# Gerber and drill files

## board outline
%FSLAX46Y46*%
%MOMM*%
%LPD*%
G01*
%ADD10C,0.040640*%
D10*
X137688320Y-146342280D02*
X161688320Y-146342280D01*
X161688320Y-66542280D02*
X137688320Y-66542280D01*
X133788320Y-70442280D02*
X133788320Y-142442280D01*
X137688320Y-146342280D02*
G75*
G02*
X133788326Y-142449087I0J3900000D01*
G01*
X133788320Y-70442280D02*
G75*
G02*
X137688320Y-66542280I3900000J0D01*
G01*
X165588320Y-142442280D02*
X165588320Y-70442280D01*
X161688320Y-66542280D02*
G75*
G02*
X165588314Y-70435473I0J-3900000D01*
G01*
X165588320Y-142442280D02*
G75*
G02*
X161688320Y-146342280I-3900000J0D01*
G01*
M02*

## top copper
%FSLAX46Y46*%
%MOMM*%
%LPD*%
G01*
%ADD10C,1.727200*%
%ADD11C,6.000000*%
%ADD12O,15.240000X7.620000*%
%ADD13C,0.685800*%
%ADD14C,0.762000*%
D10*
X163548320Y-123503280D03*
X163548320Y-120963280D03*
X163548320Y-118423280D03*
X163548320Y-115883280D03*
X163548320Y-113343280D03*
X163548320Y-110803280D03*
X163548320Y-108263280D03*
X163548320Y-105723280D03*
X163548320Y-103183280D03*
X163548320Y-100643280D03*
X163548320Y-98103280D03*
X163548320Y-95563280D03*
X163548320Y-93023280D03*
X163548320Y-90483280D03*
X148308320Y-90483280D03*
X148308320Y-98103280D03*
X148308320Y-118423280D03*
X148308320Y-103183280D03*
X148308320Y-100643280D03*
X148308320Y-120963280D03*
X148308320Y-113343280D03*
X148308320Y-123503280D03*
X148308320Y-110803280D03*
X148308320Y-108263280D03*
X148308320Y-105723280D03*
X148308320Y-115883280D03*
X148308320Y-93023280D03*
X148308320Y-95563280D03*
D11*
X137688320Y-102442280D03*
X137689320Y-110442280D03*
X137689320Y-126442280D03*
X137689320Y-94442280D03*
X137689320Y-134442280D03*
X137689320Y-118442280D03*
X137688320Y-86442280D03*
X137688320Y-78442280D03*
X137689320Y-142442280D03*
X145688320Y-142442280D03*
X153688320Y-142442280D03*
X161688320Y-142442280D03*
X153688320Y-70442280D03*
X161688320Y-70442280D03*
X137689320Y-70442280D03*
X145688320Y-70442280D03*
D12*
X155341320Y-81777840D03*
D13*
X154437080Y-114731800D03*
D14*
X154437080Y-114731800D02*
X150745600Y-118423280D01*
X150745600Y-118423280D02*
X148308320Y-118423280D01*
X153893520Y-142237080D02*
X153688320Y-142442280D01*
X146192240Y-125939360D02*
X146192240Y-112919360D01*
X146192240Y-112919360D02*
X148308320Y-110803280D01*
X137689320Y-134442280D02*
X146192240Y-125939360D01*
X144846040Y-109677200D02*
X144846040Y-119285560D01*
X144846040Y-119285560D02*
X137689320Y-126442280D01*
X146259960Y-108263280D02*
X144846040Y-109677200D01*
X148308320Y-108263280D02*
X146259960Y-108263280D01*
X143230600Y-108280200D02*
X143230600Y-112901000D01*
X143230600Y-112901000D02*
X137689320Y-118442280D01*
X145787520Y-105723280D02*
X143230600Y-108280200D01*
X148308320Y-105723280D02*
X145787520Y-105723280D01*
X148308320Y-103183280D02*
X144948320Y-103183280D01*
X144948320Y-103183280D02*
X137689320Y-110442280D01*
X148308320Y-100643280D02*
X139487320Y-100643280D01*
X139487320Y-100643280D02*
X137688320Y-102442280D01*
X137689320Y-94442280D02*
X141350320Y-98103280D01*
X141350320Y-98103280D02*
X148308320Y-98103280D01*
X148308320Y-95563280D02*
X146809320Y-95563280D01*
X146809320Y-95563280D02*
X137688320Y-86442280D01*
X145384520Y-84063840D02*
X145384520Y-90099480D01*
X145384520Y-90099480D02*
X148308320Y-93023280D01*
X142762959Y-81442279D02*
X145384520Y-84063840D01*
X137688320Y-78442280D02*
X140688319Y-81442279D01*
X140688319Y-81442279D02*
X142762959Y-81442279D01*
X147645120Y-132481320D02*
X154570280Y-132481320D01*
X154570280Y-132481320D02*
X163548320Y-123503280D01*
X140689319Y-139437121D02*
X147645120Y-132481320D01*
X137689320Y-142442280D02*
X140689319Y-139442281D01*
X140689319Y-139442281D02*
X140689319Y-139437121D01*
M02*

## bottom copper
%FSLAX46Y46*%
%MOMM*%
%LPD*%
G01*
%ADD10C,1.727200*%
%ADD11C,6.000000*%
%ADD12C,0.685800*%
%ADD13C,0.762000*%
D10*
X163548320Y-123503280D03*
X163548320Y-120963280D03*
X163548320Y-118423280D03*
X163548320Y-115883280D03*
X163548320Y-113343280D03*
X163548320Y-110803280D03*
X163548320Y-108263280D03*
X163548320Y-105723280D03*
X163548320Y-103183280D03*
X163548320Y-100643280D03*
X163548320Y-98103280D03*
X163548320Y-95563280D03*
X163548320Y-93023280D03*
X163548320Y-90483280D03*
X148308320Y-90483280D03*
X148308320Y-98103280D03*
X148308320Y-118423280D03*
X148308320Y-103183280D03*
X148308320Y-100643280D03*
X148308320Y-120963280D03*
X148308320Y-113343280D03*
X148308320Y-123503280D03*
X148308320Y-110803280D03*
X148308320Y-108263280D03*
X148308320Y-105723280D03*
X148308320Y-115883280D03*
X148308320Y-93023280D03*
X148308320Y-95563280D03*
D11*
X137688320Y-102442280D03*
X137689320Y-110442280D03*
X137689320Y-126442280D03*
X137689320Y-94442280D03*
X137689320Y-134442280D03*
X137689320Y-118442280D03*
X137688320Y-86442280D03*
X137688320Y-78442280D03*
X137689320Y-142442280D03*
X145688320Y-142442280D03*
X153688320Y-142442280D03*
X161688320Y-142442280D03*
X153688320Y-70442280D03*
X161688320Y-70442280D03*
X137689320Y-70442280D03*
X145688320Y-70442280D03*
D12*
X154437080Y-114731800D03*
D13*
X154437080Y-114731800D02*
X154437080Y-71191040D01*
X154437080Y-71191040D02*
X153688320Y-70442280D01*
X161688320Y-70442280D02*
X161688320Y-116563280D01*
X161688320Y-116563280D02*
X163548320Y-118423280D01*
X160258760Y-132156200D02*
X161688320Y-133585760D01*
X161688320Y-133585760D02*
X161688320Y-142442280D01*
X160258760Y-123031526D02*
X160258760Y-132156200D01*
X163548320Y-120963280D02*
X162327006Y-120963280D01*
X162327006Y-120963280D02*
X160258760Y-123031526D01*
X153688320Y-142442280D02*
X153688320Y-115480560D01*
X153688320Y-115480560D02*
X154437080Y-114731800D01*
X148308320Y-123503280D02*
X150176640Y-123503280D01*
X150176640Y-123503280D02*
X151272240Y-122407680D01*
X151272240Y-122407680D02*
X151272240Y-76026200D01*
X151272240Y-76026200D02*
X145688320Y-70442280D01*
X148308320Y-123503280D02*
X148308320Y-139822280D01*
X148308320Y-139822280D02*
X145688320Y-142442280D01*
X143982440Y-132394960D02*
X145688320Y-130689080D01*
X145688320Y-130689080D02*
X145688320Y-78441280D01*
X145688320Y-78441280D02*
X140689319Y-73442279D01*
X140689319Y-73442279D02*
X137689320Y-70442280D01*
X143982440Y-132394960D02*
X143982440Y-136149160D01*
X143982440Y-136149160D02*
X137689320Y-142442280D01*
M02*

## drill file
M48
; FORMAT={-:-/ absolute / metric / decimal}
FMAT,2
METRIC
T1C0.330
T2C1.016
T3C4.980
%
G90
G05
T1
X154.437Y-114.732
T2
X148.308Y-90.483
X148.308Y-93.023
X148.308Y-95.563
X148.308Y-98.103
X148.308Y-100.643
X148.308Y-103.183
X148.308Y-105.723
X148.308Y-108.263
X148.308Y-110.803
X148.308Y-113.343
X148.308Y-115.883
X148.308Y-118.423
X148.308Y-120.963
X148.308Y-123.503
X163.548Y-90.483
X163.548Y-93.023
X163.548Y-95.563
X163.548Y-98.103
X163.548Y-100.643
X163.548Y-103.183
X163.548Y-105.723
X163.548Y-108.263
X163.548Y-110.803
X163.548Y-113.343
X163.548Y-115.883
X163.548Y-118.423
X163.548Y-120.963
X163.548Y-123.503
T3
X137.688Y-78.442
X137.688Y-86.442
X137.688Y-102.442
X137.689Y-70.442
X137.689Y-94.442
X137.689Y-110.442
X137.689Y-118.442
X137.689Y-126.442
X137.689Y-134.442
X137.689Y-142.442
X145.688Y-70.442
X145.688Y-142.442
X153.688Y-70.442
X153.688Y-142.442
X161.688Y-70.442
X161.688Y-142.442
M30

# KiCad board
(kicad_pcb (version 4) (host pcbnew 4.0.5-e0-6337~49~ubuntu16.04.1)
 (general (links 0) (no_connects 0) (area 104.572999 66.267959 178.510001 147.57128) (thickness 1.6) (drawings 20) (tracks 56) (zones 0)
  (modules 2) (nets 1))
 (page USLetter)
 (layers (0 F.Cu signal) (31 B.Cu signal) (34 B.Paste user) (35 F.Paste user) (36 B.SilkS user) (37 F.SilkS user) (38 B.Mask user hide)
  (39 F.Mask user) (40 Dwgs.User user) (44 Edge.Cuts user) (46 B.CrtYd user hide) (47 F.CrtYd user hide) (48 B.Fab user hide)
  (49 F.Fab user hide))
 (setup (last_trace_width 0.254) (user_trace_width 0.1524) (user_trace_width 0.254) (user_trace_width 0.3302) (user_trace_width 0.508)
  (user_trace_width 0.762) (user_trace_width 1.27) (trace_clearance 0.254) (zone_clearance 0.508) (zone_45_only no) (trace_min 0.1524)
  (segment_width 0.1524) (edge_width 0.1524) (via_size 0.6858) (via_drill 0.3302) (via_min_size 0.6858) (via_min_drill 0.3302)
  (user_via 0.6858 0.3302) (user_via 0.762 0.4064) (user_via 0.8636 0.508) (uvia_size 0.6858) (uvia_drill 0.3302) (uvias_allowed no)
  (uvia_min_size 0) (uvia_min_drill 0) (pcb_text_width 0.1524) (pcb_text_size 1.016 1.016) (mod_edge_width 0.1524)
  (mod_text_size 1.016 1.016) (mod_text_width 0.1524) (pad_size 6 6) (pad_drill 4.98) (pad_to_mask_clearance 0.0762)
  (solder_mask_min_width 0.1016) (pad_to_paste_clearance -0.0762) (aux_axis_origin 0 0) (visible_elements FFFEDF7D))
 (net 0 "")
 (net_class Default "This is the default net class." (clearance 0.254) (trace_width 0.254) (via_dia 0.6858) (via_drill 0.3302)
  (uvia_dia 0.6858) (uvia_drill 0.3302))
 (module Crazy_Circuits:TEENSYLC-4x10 (layer F.Cu) (at 137.68832 94.44228)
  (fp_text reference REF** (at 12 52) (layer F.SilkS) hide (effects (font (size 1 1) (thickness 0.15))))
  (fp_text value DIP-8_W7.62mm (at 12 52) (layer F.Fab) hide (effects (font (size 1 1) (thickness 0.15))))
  (fp_line (start 0 51.9) (end 24 51.9) (layer Edge.Cuts) (width 0.04064))
  (fp_line (start 24 -27.9) (end 0 -27.9) (layer Edge.Cuts) (width 0.04064))
  (fp_line (start -3.9 -24) (end -3.9 48) (layer Edge.Cuts) (width 0.04064))
  (fp_arc (start 0 48) (end 0 51.9) (angle 89.9) (layer Edge.Cuts) (width 0.04064))
  (fp_arc (start 0 -24) (end -3.9 -24) (angle 90) (layer Edge.Cuts) (width 0.04064))
  (fp_line (start 27.9 48) (end 27.9 -24) (layer Edge.Cuts) (width 0.04064))
  (fp_arc (start 24 -24) (end 24 -27.9) (angle 89.9) (layer Edge.Cuts) (width 0.04064))
  (fp_arc (start 24 48) (end 27.9 48) (angle 90) (layer Edge.Cuts) (width 0.04064))
  (pad GND thru_hole circle (at 25.86 29.061 180) (size 1.7272 1.7272) (drill 1.016) (layers *.Cu *.Mask F.SilkS))
  (pad 0 thru_hole circle (at 25.86 26.521 180) (size 1.7272 1.7272) (drill 1.016) (layers *.Cu *.Mask F.SilkS))
  (pad 1 thru_hole circle (at 25.86 23.981 180) (size 1.7272 1.7272) (drill 1.016) (layers *.Cu *.Mask F.SilkS))
  (pad 2 thru_hole circle (at 25.86 21.441 180) (size 1.7272 1.7272) (drill 1.016) (layers *.Cu *.Mask F.SilkS))
  (pad 3 thru_hole circle (at 25.86 18.901 180) (size 1.7272 1.7272) (drill 1.016) (layers *.Cu *.Mask F.SilkS))
  (pad 4 thru_hole circle (at 25.86 16.361 180) (size 1.7272 1.7272) (drill 1.016) (layers *.Cu *.Mask F.SilkS))
  (pad 5 thru_hole circle (at 25.86 13.821 180) (size 1.7272 1.7272) (drill 1.016) (layers *.Cu *.Mask F.SilkS))
  (pad 6 thru_hole circle (at 25.86 11.281 180) (size 1.7272 1.7272) (drill 1.016) (layers *.Cu *.Mask F.SilkS))
  (pad 7 thru_hole circle (at 25.86 8.741 180) (size 1.7272 1.7272) (drill 1.016) (layers *.Cu *.Mask F.SilkS))
  (pad 8 thru_hole circle (at 25.86 6.201 180) (size 1.7272 1.7272) (drill 1.016) (layers *.Cu *.Mask F.SilkS))
  (pad 9 thru_hole circle (at 25.86 3.661 180) (size 1.7272 1.7272) (drill 1.016) (layers *.Cu *.Mask F.SilkS))
  (pad 10 thru_hole circle (at 25.86 1.121 180) (size 1.7272 1.7272) (drill 1.016) (layers *.Cu *.Mask F.SilkS))
  (pad 11 thru_hole circle (at 25.86 -1.419 180) (size 1.7272 1.7272) (drill 1.016) (layers *.Cu *.Mask F.SilkS))
  (pad 12 thru_hole circle (at 25.86 -3.959 180) (size 1.7272 1.7272) (drill 1.016) (layers *.Cu *.Mask F.SilkS))
  (pad 13 thru_hole circle (at 10.62 -3.959 180) (size 1.7272 1.7272) (drill 1.016) (layers *.Cu *.Mask F.SilkS))
  (pad 16 thru_hole circle (at 10.62 3.661 180) (size 1.7272 1.7272) (drill 1.016) (layers *.Cu *.Mask F.SilkS))
  (pad 3.3V thru_hole circle (at 10.62 23.981 180) (size 1.7272 1.7272) (drill 1.016) (layers *.Cu *.Mask F.SilkS))
  (pad 18 thru_hole circle (at 10.62 8.741 180) (size 1.7272 1.7272) (drill 1.016) (layers *.Cu *.Mask F.SilkS))
  (pad 17 thru_hole circle (at 10.62 6.201 180) (size 1.7272 1.7272) (drill 1.016) (layers *.Cu *.Mask F.SilkS))
  (pad G3 thru_hole circle (at 10.62 26.521 180) (size 1.7272 1.7272) (drill 1.016) (layers *.Cu *.Mask F.SilkS))
  (pad 22 thru_hole circle (at 10.62 18.901 180) (size 1.7272 1.7272) (drill 1.016) (layers *.Cu *.Mask F.SilkS))
  (pad VIN thru_hole circle (at 10.62 29.061 180) (size 1.7272 1.7272) (drill 1.016) (layers *.Cu *.Mask F.SilkS))
  (pad 21 thru_hole circle (at 10.62 16.361 180) (size 1.7272 1.7272) (drill 1.016) (layers *.Cu *.Mask F.SilkS))
  (pad 20 thru_hole circle (at 10.62 13.821 180) (size 1.7272 1.7272) (drill 1.016) (layers *.Cu *.Mask F.SilkS))
  (pad 19 thru_hole circle (at 10.62 11.281 180) (size 1.7272 1.7272) (drill 1.016) (layers *.Cu *.Mask F.SilkS))
  (pad 23 thru_hole circle (at 10.62 21.441 180) (size 1.7272 1.7272) (drill 1.016) (layers *.Cu *.Mask F.SilkS))
  (pad 14 thru_hole circle (at 10.62 -1.419 180) (size 1.7272 1.7272) (drill 1.016) (layers *.Cu *.Mask F.SilkS))
  (pad 15 thru_hole circle (at 10.62 1.121 180) (size 1.7272 1.7272) (drill 1.016) (layers *.Cu *.Mask F.SilkS))
  (pad 17 thru_hole circle (at 0 8 90) (size 6 6) (drill 4.98) (layers *.Cu *.Mask))
  (pad 18 thru_hole circle (at 0.001 16 90) (size 6 6) (drill 4.98) (layers *.Cu *.Mask))
  (pad 20 thru_hole circle (at 0.001 32 90) (size 6 6) (drill 4.98) (layers *.Cu *.Mask))
  (pad 16 thru_hole circle (at 0.001 0 90) (size 6 6) (drill 4.98) (layers *.Cu *.Mask))
  (pad 21 thru_hole circle (at 0.001 40 90) (size 6 6) (drill 4.98) (layers *.Cu *.Mask))
  (pad 19 thru_hole circle (at 0.001 24 90) (size 6 6) (drill 4.98) (layers *.Cu *.Mask))
  (pad 15 thru_hole circle (at 0 -8 90) (size 6 6) (drill 4.98) (layers *.Cu *.Mask))
  (pad 14 thru_hole circle (at 0 -16 90) (size 6 6) (drill 4.98) (layers *.Cu *.Mask))
  (pad GND thru_hole circle (at 0.001 48 90) (size 6 6) (drill 4.98) (layers *.Cu *.Mask))
  (pad VIN thru_hole circle (at 8 48 90) (size 6 6) (drill 4.98) (layers *.Cu *.Mask))
  (pad 3.3V thru_hole circle (at 16 48 90) (size 6 6) (drill 4.98) (layers *.Cu *.Mask))
  (pad 0 thru_hole circle (at 24 48 90) (size 6 6) (drill 4.98) (layers *.Cu *.Mask))
  (pad 3.3V thru_hole circle (at 16 -24 90) (size 6 6) (drill 4.98) (layers *.Cu *.Mask))
  (pad 1 thru_hole circle (at 24 -24 90) (size 6 6) (drill 4.98) (layers *.Cu *.Mask))
  (pad GND thru_hole circle (at 0.001 -24 90) (size 6 6) (drill 4.98) (layers *.Cu *.Mask))
  (pad VIN thru_hole circle (at 8 -24 90) (size 6 6) (drill 4.98) (layers *.Cu *.Mask)))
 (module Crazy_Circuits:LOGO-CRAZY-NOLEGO (layer F.Cu) (at 155.34132 85.71484)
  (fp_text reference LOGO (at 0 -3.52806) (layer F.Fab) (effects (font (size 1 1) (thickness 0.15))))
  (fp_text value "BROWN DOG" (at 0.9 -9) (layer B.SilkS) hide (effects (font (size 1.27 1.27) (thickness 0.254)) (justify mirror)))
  (pad BG smd oval (at 0 -3.937) (size 15.24 7.62) (layers F.Cu)))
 (segment (start 154.43708 114.7318) (end 154.43708 71.19104) (width 0.762) (layer B.Cu) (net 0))
 (segment (start 154.43708 71.19104) (end 153.68832 70.44228) (width 0.762) (layer B.Cu) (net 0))
 (segment (start 161.68832 70.44228) (end 161.68832 116.56328) (width 0.762) (layer B.Cu) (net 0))
 (segment (start 161.68832 116.56328) (end 163.54832 118.42328) (width 0.762) (layer B.Cu) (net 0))
 (segment (start 160.25876 132.1562) (end 161.68832 133.58576) (width 0.762) (layer B.Cu) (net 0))
 (segment (start 161.68832 133.58576) (end 161.68832 142.44228) (width 0.762) (layer B.Cu) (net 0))
 (segment (start 160.25876 123.031526) (end 160.25876 132.1562) (width 0.762) (layer B.Cu) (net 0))
 (segment (start 163.54832 120.96328) (end 162.327006 120.96328) (width 0.762) (layer B.Cu) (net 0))
 (segment (start 162.327006 120.96328) (end 160.25876 123.031526) (width 0.762) (layer B.Cu) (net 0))
 (via (at 154.43708 114.7318) (size 0.6858) (drill 0.3302) (layers F.Cu B.Cu) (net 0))
 (segment (start 153.68832 142.44228) (end 153.68832 115.48056) (width 0.762) (layer B.Cu) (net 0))
 (segment (start 153.68832 115.48056) (end 154.43708 114.7318) (width 0.762) (layer B.Cu) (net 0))
 (segment (start 154.43708 114.7318) (end 150.7456 118.42328) (width 0.762) (layer F.Cu) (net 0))
 (segment (start 150.7456 118.42328) (end 148.30832 118.42328) (width 0.762) (layer F.Cu) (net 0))
 (segment (start 148.30832 123.50328) (end 150.17664 123.50328) (width 0.762) (layer B.Cu) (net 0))
 (segment (start 150.17664 123.50328) (end 151.27224 122.40768) (width 0.762) (layer B.Cu) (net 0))
 (segment (start 151.27224 122.40768) (end 151.27224 76.0262) (width 0.762) (layer B.Cu) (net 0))
 (segment (start 151.27224 76.0262) (end 145.68832 70.44228) (width 0.762) (layer B.Cu) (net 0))
 (segment (start 148.30832 123.50328) (end 148.30832 139.82228) (width 0.762) (layer B.Cu) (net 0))
 (segment (start 148.30832 139.82228) (end 145.68832 142.44228) (width 0.762) (layer B.Cu) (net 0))
 (segment (start 143.98244 132.39496) (end 145.68832 130.68908) (width 0.762) (layer B.Cu) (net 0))
 (segment (start 145.68832 130.68908) (end 145.68832 78.44128) (width 0.762) (layer B.Cu) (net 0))
 (segment (start 145.68832 78.44128) (end 140.689319 73.442279) (width 0.762) (layer B.Cu) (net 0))
 (segment (start 140.689319 73.442279) (end 137.68932 70.44228) (width 0.762) (layer B.Cu) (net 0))
 (segment (start 153.89352 142.23708) (end 153.68832 142.44228) (width 0.762) (layer F.Cu) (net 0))
 (segment (start 143.98244 132.39496) (end 143.98244 136.14916) (width 0.762) (layer B.Cu) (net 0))
 (segment (start 143.98244 136.14916) (end 137.68932 142.44228) (width 0.762) (layer B.Cu) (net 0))
 (segment (start 146.19224 125.93936) (end 146.19224 112.91936) (width 0.762) (layer F.Cu) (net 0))
 (segment (start 146.19224 112.91936) (end 148.30832 110.80328) (width 0.762) (layer F.Cu) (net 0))
 (segment (start 137.68932 134.44228) (end 146.19224 125.93936) (width 0.762) (layer F.Cu) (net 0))
 (segment (start 144.84604 109.6772) (end 144.84604 119.28556) (width 0.762) (layer F.Cu) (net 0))
 (segment (start 144.84604 119.28556) (end 137.68932 126.44228) (width 0.762) (layer F.Cu) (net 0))
 (segment (start 146.25996 108.26328) (end 144.84604 109.6772) (width 0.762) (layer F.Cu) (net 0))
 (segment (start 148.30832 108.26328) (end 146.25996 108.26328) (width 0.762) (layer F.Cu) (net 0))
 (segment (start 143.2306 108.2802) (end 143.2306 112.901) (width 0.762) (layer F.Cu) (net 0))
 (segment (start 143.2306 112.901) (end 137.68932 118.44228) (width 0.762) (layer F.Cu) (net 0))
 (segment (start 145.78752 105.72328) (end 143.2306 108.2802) (width 0.762) (layer F.Cu) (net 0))
 (segment (start 148.30832 105.72328) (end 145.78752 105.72328) (width 0.762) (layer F.Cu) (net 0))
 (segment (start 148.30832 103.18328) (end 144.94832 103.18328) (width 0.762) (layer F.Cu) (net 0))
 (segment (start 144.94832 103.18328) (end 137.68932 110.44228) (width 0.762) (layer F.Cu) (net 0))
 (segment (start 148.30832 100.64328) (end 139.48732 100.64328) (width 0.762) (layer F.Cu) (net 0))
 (segment (start 139.48732 100.64328) (end 137.68832 102.44228) (width 0.762) (layer F.Cu) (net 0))
 (segment (start 137.68932 94.44228) (end 141.35032 98.10328) (width 0.762) (layer F.Cu) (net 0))
 (segment (start 141.35032 98.10328) (end 148.30832 98.10328) (width 0.762) (layer F.Cu) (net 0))
 (segment (start 148.30832 95.56328) (end 146.80932 95.56328) (width 0.762) (layer F.Cu) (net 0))
 (segment (start 146.80932 95.56328) (end 137.68832 86.44228) (width 0.762) (layer F.Cu) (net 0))
 (segment (start 145.38452 84.06384) (end 145.38452 90.09948) (width 0.762) (layer F.Cu) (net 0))
 (segment (start 145.38452 90.09948) (end 148.30832 93.02328) (width 0.762) (layer F.Cu) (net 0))
 (segment (start 142.762959 81.442279) (end 145.38452 84.06384) (width 0.762) (layer F.Cu) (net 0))
 (segment (start 137.68832 78.44228) (end 140.688319 81.442279) (width 0.762) (layer F.Cu) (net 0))
 (segment (start 140.688319 81.442279) (end 142.762959 81.442279) (width 0.762) (layer F.Cu) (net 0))
 (segment (start 147.64512 132.48132) (end 154.57028 132.48132) (width 0.762) (layer F.Cu) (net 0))
 (segment (start 154.57028 132.48132) (end 163.54832 123.50328) (width 0.762) (layer F.Cu) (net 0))
 (segment (start 140.689319 139.437121) (end 147.64512 132.48132) (width 0.762) (layer F.Cu) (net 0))
 (segment (start 137.68932 142.44228) (end 140.689319 139.442281) (width 0.762) (layer F.Cu) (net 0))
 (segment (start 140.689319 139.442281) (end 140.689319 139.437121) (width 0.762) (layer F.Cu) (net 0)))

